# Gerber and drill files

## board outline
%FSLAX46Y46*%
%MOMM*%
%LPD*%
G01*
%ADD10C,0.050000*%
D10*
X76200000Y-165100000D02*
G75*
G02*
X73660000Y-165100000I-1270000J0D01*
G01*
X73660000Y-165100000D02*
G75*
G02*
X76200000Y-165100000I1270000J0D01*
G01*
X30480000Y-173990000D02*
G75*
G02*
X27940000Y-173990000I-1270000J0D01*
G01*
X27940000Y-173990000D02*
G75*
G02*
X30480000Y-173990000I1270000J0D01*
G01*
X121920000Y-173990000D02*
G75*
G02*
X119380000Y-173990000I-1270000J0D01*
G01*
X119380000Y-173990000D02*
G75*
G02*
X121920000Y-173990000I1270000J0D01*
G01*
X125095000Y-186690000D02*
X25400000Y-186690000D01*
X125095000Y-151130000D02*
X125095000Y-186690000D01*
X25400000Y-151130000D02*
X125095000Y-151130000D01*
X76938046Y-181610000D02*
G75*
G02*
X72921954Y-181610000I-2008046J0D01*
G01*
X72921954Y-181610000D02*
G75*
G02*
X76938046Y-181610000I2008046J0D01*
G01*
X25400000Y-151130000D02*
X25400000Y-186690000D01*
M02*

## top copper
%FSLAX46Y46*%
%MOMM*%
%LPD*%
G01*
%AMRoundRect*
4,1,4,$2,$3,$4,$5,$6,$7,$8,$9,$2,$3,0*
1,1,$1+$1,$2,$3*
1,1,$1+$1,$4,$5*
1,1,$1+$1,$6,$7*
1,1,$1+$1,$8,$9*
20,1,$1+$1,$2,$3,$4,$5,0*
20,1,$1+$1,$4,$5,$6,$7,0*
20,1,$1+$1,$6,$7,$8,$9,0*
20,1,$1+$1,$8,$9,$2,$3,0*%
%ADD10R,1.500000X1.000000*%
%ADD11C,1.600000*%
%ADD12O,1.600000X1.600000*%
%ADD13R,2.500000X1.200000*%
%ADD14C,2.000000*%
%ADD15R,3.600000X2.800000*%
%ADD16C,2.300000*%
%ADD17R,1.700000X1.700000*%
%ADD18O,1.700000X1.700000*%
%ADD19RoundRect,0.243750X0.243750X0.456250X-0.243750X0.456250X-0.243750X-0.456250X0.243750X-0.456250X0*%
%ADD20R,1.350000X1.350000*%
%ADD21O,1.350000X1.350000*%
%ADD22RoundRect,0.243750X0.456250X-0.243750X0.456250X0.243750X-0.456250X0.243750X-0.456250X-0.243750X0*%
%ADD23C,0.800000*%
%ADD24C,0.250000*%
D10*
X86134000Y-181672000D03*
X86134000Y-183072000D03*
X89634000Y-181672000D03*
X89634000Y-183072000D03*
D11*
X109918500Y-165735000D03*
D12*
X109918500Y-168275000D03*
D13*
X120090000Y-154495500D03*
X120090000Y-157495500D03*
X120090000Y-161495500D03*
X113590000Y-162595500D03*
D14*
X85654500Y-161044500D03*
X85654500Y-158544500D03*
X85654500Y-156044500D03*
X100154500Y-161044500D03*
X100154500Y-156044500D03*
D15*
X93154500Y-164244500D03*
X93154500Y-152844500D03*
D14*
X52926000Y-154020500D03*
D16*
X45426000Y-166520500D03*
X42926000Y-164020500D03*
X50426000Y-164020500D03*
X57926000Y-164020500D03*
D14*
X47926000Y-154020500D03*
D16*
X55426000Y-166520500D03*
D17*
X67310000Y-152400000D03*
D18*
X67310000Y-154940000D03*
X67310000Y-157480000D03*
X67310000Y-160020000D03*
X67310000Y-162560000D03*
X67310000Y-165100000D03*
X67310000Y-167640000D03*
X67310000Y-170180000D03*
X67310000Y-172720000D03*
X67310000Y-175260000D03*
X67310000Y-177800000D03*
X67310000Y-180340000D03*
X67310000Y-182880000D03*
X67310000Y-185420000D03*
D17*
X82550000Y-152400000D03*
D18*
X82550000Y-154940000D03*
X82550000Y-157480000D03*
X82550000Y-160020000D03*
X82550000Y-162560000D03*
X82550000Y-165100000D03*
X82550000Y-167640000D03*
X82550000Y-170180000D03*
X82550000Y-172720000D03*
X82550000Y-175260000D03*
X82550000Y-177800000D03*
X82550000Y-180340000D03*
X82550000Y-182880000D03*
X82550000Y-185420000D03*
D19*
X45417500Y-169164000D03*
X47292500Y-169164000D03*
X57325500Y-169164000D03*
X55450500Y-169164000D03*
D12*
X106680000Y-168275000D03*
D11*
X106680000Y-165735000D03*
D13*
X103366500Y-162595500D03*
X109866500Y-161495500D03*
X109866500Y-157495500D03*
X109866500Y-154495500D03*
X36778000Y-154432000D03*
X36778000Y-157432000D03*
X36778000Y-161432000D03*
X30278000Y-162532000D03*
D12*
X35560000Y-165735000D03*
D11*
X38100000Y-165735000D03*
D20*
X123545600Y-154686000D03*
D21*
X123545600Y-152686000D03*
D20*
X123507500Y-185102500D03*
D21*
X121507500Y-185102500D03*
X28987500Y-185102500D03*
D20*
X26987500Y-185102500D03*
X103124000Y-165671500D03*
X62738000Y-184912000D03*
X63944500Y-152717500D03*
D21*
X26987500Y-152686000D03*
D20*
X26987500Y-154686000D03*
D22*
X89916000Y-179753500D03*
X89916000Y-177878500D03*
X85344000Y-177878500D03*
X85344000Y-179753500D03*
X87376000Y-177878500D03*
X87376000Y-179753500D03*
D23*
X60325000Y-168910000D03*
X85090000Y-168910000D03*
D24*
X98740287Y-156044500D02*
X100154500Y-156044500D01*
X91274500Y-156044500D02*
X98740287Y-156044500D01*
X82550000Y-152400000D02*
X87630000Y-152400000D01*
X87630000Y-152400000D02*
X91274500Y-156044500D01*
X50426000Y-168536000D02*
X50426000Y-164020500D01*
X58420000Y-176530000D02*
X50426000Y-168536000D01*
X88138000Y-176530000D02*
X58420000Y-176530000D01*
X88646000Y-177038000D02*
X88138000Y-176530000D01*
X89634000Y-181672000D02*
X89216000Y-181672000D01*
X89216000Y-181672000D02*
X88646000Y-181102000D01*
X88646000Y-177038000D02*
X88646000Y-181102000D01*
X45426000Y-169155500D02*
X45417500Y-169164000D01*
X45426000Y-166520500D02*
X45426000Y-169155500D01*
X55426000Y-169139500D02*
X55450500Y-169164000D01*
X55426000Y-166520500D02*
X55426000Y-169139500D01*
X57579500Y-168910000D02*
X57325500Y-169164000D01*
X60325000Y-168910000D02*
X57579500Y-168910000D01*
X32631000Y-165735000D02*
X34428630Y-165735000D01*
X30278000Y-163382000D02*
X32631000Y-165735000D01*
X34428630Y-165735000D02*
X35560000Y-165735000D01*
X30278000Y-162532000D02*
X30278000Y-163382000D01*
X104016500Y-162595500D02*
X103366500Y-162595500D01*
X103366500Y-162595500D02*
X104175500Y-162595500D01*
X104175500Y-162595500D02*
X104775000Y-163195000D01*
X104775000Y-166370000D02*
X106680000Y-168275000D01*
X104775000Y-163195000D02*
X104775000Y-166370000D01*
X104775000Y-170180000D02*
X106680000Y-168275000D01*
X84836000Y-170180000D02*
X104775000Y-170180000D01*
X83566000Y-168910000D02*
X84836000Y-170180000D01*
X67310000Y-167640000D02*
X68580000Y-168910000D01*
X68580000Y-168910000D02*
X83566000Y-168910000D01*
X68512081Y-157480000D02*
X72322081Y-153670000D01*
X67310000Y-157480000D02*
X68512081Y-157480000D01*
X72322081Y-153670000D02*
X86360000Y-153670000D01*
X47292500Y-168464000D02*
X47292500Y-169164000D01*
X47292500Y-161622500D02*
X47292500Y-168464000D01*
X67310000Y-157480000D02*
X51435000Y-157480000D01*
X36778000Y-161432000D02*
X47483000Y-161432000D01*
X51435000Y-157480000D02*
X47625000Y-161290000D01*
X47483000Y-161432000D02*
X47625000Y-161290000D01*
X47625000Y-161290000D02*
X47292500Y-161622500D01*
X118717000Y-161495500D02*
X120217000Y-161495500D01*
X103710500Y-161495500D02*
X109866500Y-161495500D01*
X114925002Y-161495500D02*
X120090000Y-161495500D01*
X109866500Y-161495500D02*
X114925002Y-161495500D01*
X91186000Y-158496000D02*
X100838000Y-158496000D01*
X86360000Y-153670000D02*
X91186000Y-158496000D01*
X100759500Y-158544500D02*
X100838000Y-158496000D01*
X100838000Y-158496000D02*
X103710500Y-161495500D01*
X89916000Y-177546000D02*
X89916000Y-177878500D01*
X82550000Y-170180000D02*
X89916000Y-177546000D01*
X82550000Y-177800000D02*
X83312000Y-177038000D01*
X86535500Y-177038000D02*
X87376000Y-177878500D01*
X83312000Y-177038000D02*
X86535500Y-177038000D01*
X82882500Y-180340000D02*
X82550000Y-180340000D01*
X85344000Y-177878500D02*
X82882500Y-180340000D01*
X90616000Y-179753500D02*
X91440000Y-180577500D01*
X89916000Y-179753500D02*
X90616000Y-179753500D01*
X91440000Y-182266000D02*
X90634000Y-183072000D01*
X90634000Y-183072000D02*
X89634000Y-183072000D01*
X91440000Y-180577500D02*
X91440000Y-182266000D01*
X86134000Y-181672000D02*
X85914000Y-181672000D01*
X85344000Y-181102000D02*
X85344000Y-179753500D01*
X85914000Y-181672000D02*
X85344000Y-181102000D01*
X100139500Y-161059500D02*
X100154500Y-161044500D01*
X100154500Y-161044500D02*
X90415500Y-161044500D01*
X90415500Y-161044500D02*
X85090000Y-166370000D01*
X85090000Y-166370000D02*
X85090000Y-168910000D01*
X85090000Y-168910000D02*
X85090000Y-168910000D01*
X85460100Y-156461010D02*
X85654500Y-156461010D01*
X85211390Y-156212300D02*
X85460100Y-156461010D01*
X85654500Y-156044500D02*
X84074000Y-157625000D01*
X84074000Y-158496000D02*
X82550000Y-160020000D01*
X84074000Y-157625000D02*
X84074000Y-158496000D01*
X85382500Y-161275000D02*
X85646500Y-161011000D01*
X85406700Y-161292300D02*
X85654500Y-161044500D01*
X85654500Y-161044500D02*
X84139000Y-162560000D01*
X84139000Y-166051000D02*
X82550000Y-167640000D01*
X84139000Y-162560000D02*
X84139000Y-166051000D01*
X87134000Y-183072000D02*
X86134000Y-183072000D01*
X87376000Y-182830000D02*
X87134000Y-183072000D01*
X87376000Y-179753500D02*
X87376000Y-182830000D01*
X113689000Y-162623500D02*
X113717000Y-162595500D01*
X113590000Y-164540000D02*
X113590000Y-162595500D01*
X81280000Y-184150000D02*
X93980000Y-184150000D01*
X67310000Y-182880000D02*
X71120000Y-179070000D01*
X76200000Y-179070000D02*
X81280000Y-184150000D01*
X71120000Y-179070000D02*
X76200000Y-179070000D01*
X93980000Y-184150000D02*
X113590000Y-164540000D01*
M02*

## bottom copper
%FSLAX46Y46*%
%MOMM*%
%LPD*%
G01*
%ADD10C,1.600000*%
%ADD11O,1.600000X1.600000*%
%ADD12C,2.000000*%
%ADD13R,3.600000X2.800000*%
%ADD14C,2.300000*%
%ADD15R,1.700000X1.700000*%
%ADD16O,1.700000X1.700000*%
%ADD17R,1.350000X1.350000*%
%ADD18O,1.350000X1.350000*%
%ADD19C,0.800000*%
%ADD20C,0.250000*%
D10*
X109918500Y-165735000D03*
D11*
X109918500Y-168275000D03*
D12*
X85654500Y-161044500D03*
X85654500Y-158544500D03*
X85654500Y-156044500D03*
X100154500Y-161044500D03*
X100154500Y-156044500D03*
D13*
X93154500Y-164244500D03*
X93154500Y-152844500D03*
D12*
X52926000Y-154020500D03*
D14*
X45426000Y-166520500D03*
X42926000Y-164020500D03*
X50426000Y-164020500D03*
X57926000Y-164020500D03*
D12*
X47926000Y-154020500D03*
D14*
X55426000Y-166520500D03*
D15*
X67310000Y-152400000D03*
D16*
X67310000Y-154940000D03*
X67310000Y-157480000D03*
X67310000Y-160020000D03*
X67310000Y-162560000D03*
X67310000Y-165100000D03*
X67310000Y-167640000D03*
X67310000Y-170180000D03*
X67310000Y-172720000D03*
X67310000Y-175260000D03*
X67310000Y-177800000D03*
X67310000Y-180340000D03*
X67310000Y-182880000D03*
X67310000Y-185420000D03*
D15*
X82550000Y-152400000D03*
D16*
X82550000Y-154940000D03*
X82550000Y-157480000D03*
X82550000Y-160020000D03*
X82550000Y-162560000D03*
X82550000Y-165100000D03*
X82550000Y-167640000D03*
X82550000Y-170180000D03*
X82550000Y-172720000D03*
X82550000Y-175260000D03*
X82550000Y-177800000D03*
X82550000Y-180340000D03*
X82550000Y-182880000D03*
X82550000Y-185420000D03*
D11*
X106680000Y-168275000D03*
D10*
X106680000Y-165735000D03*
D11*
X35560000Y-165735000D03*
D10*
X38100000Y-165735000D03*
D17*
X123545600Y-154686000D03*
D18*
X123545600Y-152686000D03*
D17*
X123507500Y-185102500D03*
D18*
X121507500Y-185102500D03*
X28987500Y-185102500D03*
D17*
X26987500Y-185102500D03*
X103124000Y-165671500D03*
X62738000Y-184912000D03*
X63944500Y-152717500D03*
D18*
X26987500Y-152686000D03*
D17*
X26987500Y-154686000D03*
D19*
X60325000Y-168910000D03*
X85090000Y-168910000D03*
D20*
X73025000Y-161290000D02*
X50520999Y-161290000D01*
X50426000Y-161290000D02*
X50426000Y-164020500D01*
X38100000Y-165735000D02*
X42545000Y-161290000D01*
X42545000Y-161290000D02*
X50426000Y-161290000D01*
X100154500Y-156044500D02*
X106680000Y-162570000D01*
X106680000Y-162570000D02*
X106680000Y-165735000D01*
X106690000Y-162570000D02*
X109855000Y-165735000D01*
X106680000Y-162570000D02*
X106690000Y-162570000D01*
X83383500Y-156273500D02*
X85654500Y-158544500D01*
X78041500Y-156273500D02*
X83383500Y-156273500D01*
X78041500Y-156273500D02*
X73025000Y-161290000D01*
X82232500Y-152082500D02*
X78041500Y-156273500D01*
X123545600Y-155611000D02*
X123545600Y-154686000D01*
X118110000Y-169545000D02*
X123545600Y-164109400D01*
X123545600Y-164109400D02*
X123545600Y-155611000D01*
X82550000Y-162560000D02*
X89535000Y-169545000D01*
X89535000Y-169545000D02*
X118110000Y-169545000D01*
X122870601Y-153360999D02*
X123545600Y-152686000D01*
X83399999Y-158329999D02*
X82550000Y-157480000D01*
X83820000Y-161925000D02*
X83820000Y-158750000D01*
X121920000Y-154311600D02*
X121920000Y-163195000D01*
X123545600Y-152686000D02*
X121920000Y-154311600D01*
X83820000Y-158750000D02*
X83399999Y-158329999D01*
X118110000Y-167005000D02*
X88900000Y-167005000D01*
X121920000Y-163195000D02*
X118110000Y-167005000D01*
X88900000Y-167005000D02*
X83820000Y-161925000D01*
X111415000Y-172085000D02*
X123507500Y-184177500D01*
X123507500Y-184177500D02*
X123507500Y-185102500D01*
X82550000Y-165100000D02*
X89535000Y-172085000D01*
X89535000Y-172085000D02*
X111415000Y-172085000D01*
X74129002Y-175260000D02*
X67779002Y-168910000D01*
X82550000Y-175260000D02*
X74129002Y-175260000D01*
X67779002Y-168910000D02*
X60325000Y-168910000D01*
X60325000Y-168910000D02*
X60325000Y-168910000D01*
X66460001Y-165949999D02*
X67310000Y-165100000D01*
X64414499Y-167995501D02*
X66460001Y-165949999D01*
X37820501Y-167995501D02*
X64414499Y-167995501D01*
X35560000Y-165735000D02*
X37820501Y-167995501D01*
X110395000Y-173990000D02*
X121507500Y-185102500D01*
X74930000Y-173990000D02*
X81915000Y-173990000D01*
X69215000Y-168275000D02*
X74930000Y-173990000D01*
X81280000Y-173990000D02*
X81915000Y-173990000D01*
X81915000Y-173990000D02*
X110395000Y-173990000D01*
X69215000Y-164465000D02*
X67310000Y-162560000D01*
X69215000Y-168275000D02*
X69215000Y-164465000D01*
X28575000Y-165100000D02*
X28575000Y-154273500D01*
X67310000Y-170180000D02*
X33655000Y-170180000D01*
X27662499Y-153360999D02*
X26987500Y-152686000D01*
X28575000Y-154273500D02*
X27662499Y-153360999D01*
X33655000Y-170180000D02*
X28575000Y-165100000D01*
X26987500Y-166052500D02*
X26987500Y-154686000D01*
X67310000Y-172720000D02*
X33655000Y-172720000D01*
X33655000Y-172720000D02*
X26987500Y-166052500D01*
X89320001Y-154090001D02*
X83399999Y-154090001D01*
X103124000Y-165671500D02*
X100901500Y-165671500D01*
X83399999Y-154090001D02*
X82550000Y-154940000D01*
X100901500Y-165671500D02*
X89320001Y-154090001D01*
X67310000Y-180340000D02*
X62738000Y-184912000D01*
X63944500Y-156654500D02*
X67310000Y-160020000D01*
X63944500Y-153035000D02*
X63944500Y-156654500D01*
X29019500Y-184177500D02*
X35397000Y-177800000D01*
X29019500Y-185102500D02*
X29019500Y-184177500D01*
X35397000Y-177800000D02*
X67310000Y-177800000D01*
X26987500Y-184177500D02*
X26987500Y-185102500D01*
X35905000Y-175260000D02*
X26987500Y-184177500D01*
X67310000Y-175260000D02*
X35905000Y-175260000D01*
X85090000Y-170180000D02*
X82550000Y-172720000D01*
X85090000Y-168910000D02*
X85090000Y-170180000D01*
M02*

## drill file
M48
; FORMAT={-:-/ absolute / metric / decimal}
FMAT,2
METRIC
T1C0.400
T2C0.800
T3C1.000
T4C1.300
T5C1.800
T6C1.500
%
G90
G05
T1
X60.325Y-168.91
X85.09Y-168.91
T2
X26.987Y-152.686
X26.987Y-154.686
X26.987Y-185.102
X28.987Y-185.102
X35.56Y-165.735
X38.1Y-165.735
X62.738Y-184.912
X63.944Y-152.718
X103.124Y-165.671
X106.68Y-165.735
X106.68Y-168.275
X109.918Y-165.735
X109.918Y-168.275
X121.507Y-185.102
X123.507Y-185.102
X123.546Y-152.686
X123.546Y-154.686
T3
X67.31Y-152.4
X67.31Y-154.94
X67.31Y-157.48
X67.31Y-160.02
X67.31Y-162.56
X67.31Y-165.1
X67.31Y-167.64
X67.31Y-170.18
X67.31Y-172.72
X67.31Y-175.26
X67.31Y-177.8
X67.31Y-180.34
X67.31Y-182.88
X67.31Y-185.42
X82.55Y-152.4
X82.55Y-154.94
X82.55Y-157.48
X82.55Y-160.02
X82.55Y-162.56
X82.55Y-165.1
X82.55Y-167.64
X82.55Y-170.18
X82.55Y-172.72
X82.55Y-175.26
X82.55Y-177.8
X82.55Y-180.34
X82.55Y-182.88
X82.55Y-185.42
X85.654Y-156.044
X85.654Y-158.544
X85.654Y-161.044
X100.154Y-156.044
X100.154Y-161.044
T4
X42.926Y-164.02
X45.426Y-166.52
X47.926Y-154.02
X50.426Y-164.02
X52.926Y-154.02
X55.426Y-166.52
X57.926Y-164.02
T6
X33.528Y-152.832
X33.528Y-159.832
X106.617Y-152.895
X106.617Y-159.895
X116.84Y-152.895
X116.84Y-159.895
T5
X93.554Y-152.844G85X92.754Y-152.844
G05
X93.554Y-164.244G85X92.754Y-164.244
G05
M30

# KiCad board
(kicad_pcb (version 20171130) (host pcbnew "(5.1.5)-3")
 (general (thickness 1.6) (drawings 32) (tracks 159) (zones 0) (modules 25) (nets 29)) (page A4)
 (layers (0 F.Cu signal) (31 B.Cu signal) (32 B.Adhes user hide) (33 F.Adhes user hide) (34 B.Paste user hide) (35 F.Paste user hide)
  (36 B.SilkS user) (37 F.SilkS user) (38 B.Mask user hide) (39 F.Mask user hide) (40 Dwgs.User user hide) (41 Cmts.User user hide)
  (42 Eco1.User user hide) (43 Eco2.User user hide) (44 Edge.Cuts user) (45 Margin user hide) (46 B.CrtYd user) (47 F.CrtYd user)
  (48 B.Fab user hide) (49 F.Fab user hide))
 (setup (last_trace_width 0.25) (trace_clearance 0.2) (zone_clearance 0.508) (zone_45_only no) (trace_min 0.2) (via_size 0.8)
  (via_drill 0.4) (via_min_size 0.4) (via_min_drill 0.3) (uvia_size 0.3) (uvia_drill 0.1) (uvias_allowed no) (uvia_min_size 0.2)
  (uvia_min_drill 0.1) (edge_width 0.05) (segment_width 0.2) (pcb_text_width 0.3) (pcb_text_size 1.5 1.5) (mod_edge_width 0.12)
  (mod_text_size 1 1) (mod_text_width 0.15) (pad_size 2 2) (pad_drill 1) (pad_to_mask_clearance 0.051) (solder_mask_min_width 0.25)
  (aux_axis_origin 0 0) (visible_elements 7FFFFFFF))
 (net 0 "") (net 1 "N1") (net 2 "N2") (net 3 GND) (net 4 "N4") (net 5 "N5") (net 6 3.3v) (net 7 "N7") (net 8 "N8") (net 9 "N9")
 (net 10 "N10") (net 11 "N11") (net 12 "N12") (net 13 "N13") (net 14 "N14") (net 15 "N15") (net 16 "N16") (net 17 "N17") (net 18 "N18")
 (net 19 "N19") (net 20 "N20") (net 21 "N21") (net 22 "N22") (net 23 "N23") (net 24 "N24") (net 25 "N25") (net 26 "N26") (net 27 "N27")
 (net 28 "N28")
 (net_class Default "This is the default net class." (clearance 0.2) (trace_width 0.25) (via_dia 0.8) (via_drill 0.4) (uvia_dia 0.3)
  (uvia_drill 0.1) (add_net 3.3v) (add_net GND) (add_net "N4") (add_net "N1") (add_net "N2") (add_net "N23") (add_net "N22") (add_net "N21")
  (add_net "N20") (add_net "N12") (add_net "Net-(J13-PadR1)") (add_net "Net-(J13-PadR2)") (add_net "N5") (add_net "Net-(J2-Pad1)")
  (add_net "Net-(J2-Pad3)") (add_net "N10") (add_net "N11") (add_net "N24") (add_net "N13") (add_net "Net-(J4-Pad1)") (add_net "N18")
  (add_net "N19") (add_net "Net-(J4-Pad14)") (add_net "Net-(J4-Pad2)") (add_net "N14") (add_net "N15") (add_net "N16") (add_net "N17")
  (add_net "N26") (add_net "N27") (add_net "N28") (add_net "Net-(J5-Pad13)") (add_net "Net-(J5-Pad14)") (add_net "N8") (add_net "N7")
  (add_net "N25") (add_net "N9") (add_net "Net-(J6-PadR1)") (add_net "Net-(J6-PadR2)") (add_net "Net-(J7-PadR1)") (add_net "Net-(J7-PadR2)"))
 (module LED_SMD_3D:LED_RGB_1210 (layer F.Cu) (at 87.884 182.372 180)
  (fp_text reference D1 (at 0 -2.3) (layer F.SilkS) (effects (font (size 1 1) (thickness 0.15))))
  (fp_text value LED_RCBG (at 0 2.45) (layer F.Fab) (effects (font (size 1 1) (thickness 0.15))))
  (pad 3 smd rect (at 1.75 0.7) (size 1.5 1) (layers F.Cu F.Paste F.Mask) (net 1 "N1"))
  (pad 4 smd rect (at 1.75 -0.7) (size 1.5 1) (layers F.Cu F.Paste F.Mask) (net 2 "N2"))
  (pad 2 smd rect (at -1.75 0.7) (size 1.5 1) (layers F.Cu F.Paste F.Mask) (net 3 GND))
  (pad 1 smd rect (at -1.75 -0.7) (size 1.5 1) (layers F.Cu F.Paste F.Mask) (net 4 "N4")))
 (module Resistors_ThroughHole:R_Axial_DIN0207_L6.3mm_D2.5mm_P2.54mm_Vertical (layer F.Cu) (at 109.9185 165.735 270)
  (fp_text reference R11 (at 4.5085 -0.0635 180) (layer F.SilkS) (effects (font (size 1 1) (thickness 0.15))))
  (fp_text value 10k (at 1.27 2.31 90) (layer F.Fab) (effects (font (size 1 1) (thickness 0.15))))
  (pad 1 thru_hole circle (at 0 0 270) (size 1.6 1.6) (drill 0.8) (layers *.Cu *.Mask) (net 3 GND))
  (pad 2 thru_hole oval (at 2.54 0 270) (size 1.6 1.6) (drill 0.8) (layers *.Cu *.Mask) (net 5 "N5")))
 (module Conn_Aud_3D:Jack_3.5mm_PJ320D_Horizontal (layer F.Cu) (at 116.84 157.6705 270)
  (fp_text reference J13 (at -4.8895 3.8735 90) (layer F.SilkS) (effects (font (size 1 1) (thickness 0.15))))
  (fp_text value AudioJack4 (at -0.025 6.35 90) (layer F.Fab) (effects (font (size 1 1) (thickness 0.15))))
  (pad "" np_thru_hole circle (at 2.225 0 270) (size 1.5 1.5) (drill 1.5) (layers *.Cu *.Mask))
  (pad "" np_thru_hole circle (at -4.775 0 270) (size 1.5 1.5) (drill 1.5) (layers *.Cu *.Mask))
  (pad R2 smd rect (at -3.175 -3.25 270) (size 1.2 2.5) (layers F.Cu F.Paste F.Mask))
  (pad R1 smd rect (at -0.175 -3.25 270) (size 1.2 2.5) (layers F.Cu F.Paste F.Mask))
  (pad T smd rect (at 3.825 -3.25 270) (size 1.2 2.5) (layers F.Cu F.Paste F.Mask) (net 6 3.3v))
  (pad S smd rect (at 4.925 3.25 270) (size 1.2 2.5) (layers F.Cu F.Paste F.Mask) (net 5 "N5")))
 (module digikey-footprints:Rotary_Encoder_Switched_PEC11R (layer F.Cu) (at 93.1545 152.8445 270)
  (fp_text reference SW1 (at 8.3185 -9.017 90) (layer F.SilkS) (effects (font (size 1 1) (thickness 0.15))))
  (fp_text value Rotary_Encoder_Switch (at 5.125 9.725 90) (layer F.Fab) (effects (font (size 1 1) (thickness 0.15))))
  (pad B thru_hole circle (at 8.2 7.5 270) (size 2 2) (drill 1) (layers *.Cu *.Mask) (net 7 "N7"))
  (pad C thru_hole circle (at 5.7 7.5 270) (size 2 2) (drill 1) (layers *.Cu *.Mask) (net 3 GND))
  (pad A thru_hole circle (at 3.2 7.5 270) (size 2 2) (drill 1) (layers *.Cu *.Mask) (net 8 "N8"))
  (pad S2 thru_hole circle (at 8.2 -7 270) (size 2 2) (drill 1) (layers *.Cu *.Mask) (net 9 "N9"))
  (pad S1 thru_hole circle (at 3.2 -7 270) (size 2 2) (drill 1) (layers *.Cu *.Mask) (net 3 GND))
  (pad 3 thru_hole rect (at 11.4 0 270) (size 2.8 3.6) (drill oval 1.8 2.6) (layers *.Cu *.Mask))
  (pad 3 thru_hole rect (at 0 0 270) (size 2.8 3.6) (drill oval 1.8 2.6) (layers *.Cu *.Mask)))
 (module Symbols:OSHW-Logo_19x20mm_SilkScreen (layer F.Cu) (at 110.49 175.895)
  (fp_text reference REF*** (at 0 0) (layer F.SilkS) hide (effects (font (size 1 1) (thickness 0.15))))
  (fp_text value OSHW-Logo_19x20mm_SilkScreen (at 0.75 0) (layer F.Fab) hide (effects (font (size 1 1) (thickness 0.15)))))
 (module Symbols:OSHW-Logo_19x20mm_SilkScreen (layer B.Cu) (at 110.49 175.895 180)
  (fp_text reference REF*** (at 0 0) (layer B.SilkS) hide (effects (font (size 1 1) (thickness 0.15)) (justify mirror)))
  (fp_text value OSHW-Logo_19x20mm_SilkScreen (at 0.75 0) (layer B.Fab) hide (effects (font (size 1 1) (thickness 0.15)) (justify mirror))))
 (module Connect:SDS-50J (layer F.Cu) (at 42.926 164.0205)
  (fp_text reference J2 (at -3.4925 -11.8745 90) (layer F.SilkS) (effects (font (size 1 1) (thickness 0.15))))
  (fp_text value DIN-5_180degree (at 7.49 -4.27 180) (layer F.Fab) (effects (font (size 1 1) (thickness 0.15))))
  (pad "" thru_hole circle (at 10 -10) (size 2 2) (drill 1.3) (layers *.Cu *.Mask))
  (pad 4 thru_hole circle (at 2.5 2.5) (size 2.3 2.3) (drill 1.3) (layers *.Cu *.Mask) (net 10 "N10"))
  (pad 1 thru_hole circle (at 0 0) (size 2.3 2.3) (drill 1.3) (layers *.Cu *.Mask))
  (pad 2 thru_hole circle (at 7.5 0) (size 2.3 2.3) (drill 1.3) (layers *.Cu *.Mask) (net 3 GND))
  (pad 3 thru_hole circle (at 15 0) (size 2.3 2.3) (drill 1.3) (layers *.Cu *.Mask))
  (pad "" thru_hole circle (at 5 -10) (size 2 2) (drill 1.3) (layers *.Cu *.Mask))
  (pad 5 thru_hole circle (at 12.5 2.5) (size 2.3 2.3) (drill 1.3) (layers *.Cu *.Mask) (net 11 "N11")))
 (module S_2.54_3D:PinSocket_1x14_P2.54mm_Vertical (layer F.Cu) (at 67.31 152.4)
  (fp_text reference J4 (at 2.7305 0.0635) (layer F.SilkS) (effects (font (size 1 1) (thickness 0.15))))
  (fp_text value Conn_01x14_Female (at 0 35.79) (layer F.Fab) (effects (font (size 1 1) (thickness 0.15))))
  (pad 1 thru_hole rect (at 0 0) (size 1.7 1.7) (drill 1) (layers *.Cu *.Mask))
  (pad 2 thru_hole oval (at 0 2.54) (size 1.7 1.7) (drill 1) (layers *.Cu *.Mask))
  (pad 3 thru_hole oval (at 0 5.08) (size 1.7 1.7) (drill 1) (layers *.Cu *.Mask) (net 6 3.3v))
  (pad 4 thru_hole oval (at 0 7.62) (size 1.7 1.7) (drill 1) (layers *.Cu *.Mask) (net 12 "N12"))
  (pad 5 thru_hole oval (at 0 10.16) (size 1.7 1.7) (drill 1) (layers *.Cu *.Mask) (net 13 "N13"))
  (pad 6 thru_hole oval (at 0 12.7) (size 1.7 1.7) (drill 1) (layers *.Cu *.Mask) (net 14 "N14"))
  (pad 7 thru_hole oval (at 0 15.24) (size 1.7 1.7) (drill 1) (layers *.Cu *.Mask) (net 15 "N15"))
  (pad 8 thru_hole oval (at 0 17.78) (size 1.7 1.7) (drill 1) (layers *.Cu *.Mask) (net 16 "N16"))
  (pad 9 thru_hole oval (at 0 20.32) (size 1.7 1.7) (drill 1) (layers *.Cu *.Mask) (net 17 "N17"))
  (pad 10 thru_hole oval (at 0 22.86) (size 1.7 1.7) (drill 1) (layers *.Cu *.Mask) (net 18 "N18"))
  (pad 11 thru_hole oval (at 0 25.4) (size 1.7 1.7) (drill 1) (layers *.Cu *.Mask) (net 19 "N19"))
  (pad 12 thru_hole oval (at 0 27.94) (size 1.7 1.7) (drill 1) (layers *.Cu *.Mask) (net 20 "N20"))
  (pad 13 thru_hole oval (at 0 30.48) (size 1.7 1.7) (drill 1) (layers *.Cu *.Mask) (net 5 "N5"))
  (pad 14 thru_hole oval (at 0 33.02) (size 1.7 1.7) (drill 1) (layers *.Cu *.Mask)))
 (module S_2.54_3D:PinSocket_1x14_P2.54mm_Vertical (layer F.Cu) (at 82.55 152.4)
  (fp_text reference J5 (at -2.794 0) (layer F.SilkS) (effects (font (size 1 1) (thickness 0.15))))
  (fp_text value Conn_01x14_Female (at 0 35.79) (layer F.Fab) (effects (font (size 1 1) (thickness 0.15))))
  (pad 1 thru_hole rect (at 0 0) (size 1.7 1.7) (drill 1) (layers *.Cu *.Mask) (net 3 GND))
  (pad 2 thru_hole oval (at 0 2.54) (size 1.7 1.7) (drill 1) (layers *.Cu *.Mask) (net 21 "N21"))
  (pad 3 thru_hole oval (at 0 5.08) (size 1.7 1.7) (drill 1) (layers *.Cu *.Mask) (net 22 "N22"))
  (pad 4 thru_hole oval (at 0 7.62) (size 1.7 1.7) (drill 1) (layers *.Cu *.Mask) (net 8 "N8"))
  (pad 5 thru_hole oval (at 0 10.16) (size 1.7 1.7) (drill 1) (layers *.Cu *.Mask) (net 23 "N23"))
  (pad 6 thru_hole oval (at 0 12.7) (size 1.7 1.7) (drill 1) (layers *.Cu *.Mask) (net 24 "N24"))
  (pad 7 thru_hole oval (at 0 15.24) (size 1.7 1.7) (drill 1) (layers *.Cu *.Mask) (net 7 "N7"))
  (pad 8 thru_hole oval (at 0 17.78) (size 1.7 1.7) (drill 1) (layers *.Cu *.Mask) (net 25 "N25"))
  (pad 9 thru_hole oval (at 0 20.32) (size 1.7 1.7) (drill 1) (layers *.Cu *.Mask) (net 9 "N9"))
  (pad 10 thru_hole oval (at 0 22.86) (size 1.7 1.7) (drill 1) (layers *.Cu *.Mask) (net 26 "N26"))
  (pad 11 thru_hole oval (at 0 25.4) (size 1.7 1.7) (drill 1) (layers *.Cu *.Mask) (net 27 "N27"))
  (pad 12 thru_hole oval (at 0 27.94) (size 1.7 1.7) (drill 1) (layers *.Cu *.Mask) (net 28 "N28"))
  (pad 13 thru_hole oval (at 0 30.48) (size 1.7 1.7) (drill 1) (layers *.Cu *.Mask))
  (pad 14 thru_hole oval (at 0 33.02) (size 1.7 1.7) (drill 1) (layers *.Cu *.Mask)))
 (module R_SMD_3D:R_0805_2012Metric (layer F.Cu) (at 46.355 169.164 180)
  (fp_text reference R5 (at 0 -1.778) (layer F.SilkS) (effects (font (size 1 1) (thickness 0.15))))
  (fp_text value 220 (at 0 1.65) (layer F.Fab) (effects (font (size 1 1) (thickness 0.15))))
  (pad 2 smd roundrect (at 0.9375 0 180) (size 0.975 1.4) (layers F.Cu F.Paste F.Mask) (roundrect_rratio 0.25) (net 10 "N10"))
  (pad 1 smd roundrect (at -0.9375 0 180) (size 0.975 1.4) (layers F.Cu F.Paste F.Mask) (roundrect_rratio 0.25) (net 6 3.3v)))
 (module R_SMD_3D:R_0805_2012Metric (layer F.Cu) (at 56.388 169.164 180)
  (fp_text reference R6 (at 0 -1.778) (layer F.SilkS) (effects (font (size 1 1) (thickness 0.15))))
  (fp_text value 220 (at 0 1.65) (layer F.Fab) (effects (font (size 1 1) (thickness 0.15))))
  (pad 1 smd roundrect (at -0.9375 0 180) (size 0.975 1.4) (layers F.Cu F.Paste F.Mask) (roundrect_rratio 0.25) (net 26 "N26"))
  (pad 2 smd roundrect (at 0.9375 0 180) (size 0.975 1.4) (layers F.Cu F.Paste F.Mask) (roundrect_rratio 0.25) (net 11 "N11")))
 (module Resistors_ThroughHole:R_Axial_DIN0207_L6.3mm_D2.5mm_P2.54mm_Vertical (layer F.Cu) (at 106.68 165.735 270)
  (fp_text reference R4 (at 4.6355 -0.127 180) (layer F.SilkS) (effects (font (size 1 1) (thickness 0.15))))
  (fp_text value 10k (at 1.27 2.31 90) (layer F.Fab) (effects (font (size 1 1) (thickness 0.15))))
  (pad 2 thru_hole oval (at 2.54 0 270) (size 1.6 1.6) (drill 0.8) (layers *.Cu *.Mask) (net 15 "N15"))
  (pad 1 thru_hole circle (at 0 0 270) (size 1.6 1.6) (drill 0.8) (layers *.Cu *.Mask) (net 3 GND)))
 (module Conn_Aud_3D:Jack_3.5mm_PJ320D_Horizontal (layer F.Cu) (at 106.6165 157.6705 270)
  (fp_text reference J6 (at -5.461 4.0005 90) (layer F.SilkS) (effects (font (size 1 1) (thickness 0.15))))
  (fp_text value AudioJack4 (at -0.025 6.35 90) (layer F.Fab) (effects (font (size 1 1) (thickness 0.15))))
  (pad S smd rect (at 4.925 3.25 270) (size 1.2 2.5) (layers F.Cu F.Paste F.Mask) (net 15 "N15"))
  (pad T smd rect (at 3.825 -3.25 270) (size 1.2 2.5) (layers F.Cu F.Paste F.Mask) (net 6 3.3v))
  (pad R1 smd rect (at -0.175 -3.25 270) (size 1.2 2.5) (layers F.Cu F.Paste F.Mask))
  (pad R2 smd rect (at -3.175 -3.25 270) (size 1.2 2.5) (layers F.Cu F.Paste F.Mask))
  (pad "" np_thru_hole circle (at -4.775 0 270) (size 1.5 1.5) (drill 1.5) (layers *.Cu *.Mask))
  (pad "" np_thru_hole circle (at 2.225 0 270) (size 1.5 1.5) (drill 1.5) (layers *.Cu *.Mask)))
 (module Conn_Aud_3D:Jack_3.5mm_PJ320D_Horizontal (layer F.Cu) (at 33.528 157.607 270)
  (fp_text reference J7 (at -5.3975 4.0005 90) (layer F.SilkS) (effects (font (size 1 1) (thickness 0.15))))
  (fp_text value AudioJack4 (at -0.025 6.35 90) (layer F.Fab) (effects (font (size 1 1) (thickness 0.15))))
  (pad "" np_thru_hole circle (at 2.225 0 270) (size 1.5 1.5) (drill 1.5) (layers *.Cu *.Mask))
  (pad "" np_thru_hole circle (at -4.775 0 270) (size 1.5 1.5) (drill 1.5) (layers *.Cu *.Mask))
  (pad R2 smd rect (at -3.175 -3.25 270) (size 1.2 2.5) (layers F.Cu F.Paste F.Mask))
  (pad R1 smd rect (at -0.175 -3.25 270) (size 1.2 2.5) (layers F.Cu F.Paste F.Mask))
  (pad T smd rect (at 3.825 -3.25 270) (size 1.2 2.5) (layers F.Cu F.Paste F.Mask) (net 6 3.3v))
  (pad S smd rect (at 4.925 3.25 270) (size 1.2 2.5) (layers F.Cu F.Paste F.Mask) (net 14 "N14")))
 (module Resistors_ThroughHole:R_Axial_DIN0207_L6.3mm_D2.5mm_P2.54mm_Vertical (layer F.Cu) (at 38.1 165.735 180)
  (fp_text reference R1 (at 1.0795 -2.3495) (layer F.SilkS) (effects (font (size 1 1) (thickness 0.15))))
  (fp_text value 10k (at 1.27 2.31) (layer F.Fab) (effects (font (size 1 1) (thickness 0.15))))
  (pad 2 thru_hole oval (at 2.54 0 180) (size 1.6 1.6) (drill 0.8) (layers *.Cu *.Mask) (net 14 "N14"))
  (pad 1 thru_hole circle (at 0 0 180) (size 1.6 1.6) (drill 0.8) (layers *.Cu *.Mask) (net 3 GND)))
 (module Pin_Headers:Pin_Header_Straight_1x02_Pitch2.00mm (layer F.Cu) (at 123.5456 154.686 180)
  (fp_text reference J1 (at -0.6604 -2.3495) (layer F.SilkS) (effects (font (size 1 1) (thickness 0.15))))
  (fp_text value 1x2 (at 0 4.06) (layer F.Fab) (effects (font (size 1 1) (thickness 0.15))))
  (pad 1 thru_hole rect (at 0 0 180) (size 1.35 1.35) (drill 0.8) (layers *.Cu *.Mask) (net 23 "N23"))
  (pad 2 thru_hole oval (at 0 2 180) (size 1.35 1.35) (drill 0.8) (layers *.Cu *.Mask) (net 22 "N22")))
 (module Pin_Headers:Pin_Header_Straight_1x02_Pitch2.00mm (layer F.Cu) (at 123.5075 185.1025 270)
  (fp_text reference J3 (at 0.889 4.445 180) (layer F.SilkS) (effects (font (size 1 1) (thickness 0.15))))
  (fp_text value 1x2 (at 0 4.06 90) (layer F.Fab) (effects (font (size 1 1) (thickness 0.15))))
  (pad 1 thru_hole rect (at 0 0 270) (size 1.35 1.35) (drill 0.8) (layers *.Cu *.Mask) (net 24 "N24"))
  (pad 2 thru_hole oval (at 0 2 270) (size 1.35 1.35) (drill 0.8) (layers *.Cu *.Mask) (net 13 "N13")))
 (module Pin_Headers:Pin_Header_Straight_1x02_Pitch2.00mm (layer F.Cu) (at 26.9875 185.1025 90)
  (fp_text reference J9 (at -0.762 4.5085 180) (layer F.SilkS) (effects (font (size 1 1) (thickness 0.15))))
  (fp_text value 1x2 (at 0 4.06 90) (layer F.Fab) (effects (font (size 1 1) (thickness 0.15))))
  (pad 2 thru_hole oval (at 0 2 90) (size 1.35 1.35) (drill 0.8) (layers *.Cu *.Mask) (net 19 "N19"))
  (pad 1 thru_hole rect (at 0 0 90) (size 1.35 1.35) (drill 0.8) (layers *.Cu *.Mask) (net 18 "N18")))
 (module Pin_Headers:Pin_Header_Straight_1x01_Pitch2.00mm (layer F.Cu) (at 103.124 165.6715)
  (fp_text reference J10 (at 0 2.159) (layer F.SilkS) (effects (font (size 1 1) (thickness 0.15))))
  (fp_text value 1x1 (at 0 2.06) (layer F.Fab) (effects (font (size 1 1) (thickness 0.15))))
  (pad 1 thru_hole rect (at 0 0) (size 1.35 1.35) (drill 0.8) (layers *.Cu *.Mask) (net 21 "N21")))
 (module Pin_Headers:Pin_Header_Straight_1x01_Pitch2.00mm (layer F.Cu) (at 62.738 184.912)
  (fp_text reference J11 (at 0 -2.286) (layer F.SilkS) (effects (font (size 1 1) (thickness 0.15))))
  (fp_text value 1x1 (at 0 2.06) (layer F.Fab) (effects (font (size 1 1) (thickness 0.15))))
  (pad 1 thru_hole rect (at 0 0) (size 1.35 1.35) (drill 0.8) (layers *.Cu *.Mask) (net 20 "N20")))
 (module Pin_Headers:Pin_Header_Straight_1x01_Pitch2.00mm (layer F.Cu) (at 63.9445 152.7175)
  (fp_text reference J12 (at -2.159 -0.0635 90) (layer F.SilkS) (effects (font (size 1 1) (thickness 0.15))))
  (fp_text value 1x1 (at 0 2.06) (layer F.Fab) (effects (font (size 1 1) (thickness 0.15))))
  (pad 1 thru_hole rect (at 0 0) (size 1.35 1.35) (drill 0.8) (layers *.Cu *.Mask) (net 12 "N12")))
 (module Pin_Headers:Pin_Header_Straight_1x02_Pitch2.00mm (layer F.Cu) (at 26.9875 154.686 180)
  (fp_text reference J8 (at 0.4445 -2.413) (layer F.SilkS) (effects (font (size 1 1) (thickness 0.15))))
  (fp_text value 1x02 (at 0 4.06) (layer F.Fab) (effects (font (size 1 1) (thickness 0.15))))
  (pad 2 thru_hole oval (at 0 2 180) (size 1.35 1.35) (drill 0.8) (layers *.Cu *.Mask) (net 16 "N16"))
  (pad 1 thru_hole rect (at 0 0 180) (size 1.35 1.35) (drill 0.8) (layers *.Cu *.Mask) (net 17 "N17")))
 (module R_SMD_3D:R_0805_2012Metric (layer F.Cu) (at 89.916 178.816 90)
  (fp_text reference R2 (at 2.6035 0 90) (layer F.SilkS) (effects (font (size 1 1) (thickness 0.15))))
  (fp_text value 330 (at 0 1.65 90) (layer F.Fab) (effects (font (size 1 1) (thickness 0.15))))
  (pad 1 smd roundrect (at -0.9375 0 90) (size 0.975 1.4) (layers F.Cu F.Paste F.Mask) (roundrect_rratio 0.25) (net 4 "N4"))
  (pad 2 smd roundrect (at 0.9375 0 90) (size 0.975 1.4) (layers F.Cu F.Paste F.Mask) (roundrect_rratio 0.25) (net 25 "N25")))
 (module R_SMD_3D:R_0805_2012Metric (layer F.Cu) (at 85.344 178.816 90)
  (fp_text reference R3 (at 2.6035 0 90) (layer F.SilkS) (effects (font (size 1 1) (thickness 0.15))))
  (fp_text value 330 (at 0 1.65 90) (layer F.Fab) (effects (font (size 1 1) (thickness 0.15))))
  (pad 2 smd roundrect (at 0.9375 0 90) (size 0.975 1.4) (layers F.Cu F.Paste F.Mask) (roundrect_rratio 0.25) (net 28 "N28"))
  (pad 1 smd roundrect (at -0.9375 0 90) (size 0.975 1.4) (layers F.Cu F.Paste F.Mask) (roundrect_rratio 0.25) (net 1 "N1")))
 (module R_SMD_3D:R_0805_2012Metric (layer F.Cu) (at 87.376 178.816 90)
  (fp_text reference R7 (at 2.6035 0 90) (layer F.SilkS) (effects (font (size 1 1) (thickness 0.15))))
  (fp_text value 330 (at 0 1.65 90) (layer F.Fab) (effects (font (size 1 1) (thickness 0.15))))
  (pad 2 smd roundrect (at 0.9375 0 90) (size 0.975 1.4) (layers F.Cu F.Paste F.Mask) (roundrect_rratio 0.25) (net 27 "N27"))
  (pad 1 smd roundrect (at -0.9375 0 90) (size 0.975 1.4) (layers F.Cu F.Paste F.Mask) (roundrect_rratio 0.25) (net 2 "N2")))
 (gr_circle (center 74.93 165.1) (end 76.2 165.1) (layer Edge.Cuts) (width 0.05))
 (gr_circle (center 29.21 173.99) (end 27.94 173.99) (layer Edge.Cuts) (width 0.05))
 (gr_circle (center 120.65 173.99) (end 121.92 173.99) (layer Edge.Cuts) (width 0.05))
 (gr_line (start 125.095 186.69) (end 25.4 186.69) (layer Edge.Cuts) (width 0.05))
 (gr_line (start 125.095 151.13) (end 125.095 186.69) (layer Edge.Cuts) (width 0.05))
 (gr_line (start 25.4 151.13) (end 125.095 151.13) (layer Edge.Cuts) (width 0.05))
 (gr_circle (center 74.93 181.61) (end 76.835 180.975) (layer Edge.Cuts) (width 0.05))
 (gr_line (start 25.4 151.13) (end 25.4 186.69) (layer Edge.Cuts) (width 0.05))
 (segment (start 98.740287 156.0445) (end 100.1545 156.0445) (width 0.25) (layer F.Cu) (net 3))
 (segment (start 91.2745 156.0445) (end 98.740287 156.0445) (width 0.25) (layer F.Cu) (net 3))
 (segment (start 82.55 152.4) (end 87.63 152.4) (width 0.25) (layer F.Cu) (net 3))
 (segment (start 87.63 152.4) (end 91.2745 156.0445) (width 0.25) (layer F.Cu) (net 3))
 (segment (start 73.025 161.29) (end 50.520999 161.29) (width 0.25) (layer B.Cu) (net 3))
 (segment (start 50.426 161.29) (end 50.426 164.0205) (width 0.25) (layer B.Cu) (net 3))
 (segment (start 38.1 165.735) (end 42.545 161.29) (width 0.25) (layer B.Cu) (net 3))
 (segment (start 42.545 161.29) (end 50.426 161.29) (width 0.25) (layer B.Cu) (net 3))
 (segment (start 100.1545 156.0445) (end 106.68 162.57) (width 0.25) (layer B.Cu) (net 3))
 (segment (start 106.68 162.57) (end 106.68 165.735) (width 0.25) (layer B.Cu) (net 3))
 (segment (start 106.69 162.57) (end 109.855 165.735) (width 0.25) (layer B.Cu) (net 3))
 (segment (start 106.68 162.57) (end 106.69 162.57) (width 0.25) (layer B.Cu) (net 3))
 (segment (start 83.3835 156.2735) (end 85.6545 158.5445) (width 0.25) (layer B.Cu) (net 3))
 (segment (start 78.0415 156.2735) (end 83.3835 156.2735) (width 0.25) (layer B.Cu) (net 3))
 (segment (start 78.0415 156.2735) (end 73.025 161.29) (width 0.25) (layer B.Cu) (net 3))
 (segment (start 82.2325 152.0825) (end 78.0415 156.2735) (width 0.25) (layer B.Cu) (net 3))
 (segment (start 50.426 168.536) (end 50.426 164.0205) (width 0.25) (layer F.Cu) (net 3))
 (segment (start 58.42 176.53) (end 50.426 168.536) (width 0.25) (layer F.Cu) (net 3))
 (segment (start 88.138 176.53) (end 58.42 176.53) (width 0.25) (layer F.Cu) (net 3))
 (segment (start 88.646 177.038) (end 88.138 176.53) (width 0.25) (layer F.Cu) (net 3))
 (segment (start 89.634 181.672) (end 89.216 181.672) (width 0.25) (layer F.Cu) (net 3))
 (segment (start 89.216 181.672) (end 88.646 181.102) (width 0.25) (layer F.Cu) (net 3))
 (segment (start 88.646 177.038) (end 88.646 181.102) (width 0.25) (layer F.Cu) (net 3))
 (segment (start 123.5456 155.611) (end 123.5456 154.686) (width 0.25) (layer B.Cu) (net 23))
 (segment (start 118.11 169.545) (end 123.5456 164.1094) (width 0.25) (layer B.Cu) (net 23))
 (segment (start 123.5456 164.1094) (end 123.5456 155.611) (width 0.25) (layer B.Cu) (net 23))
 (segment (start 82.55 162.56) (end 89.535 169.545) (width 0.25) (layer B.Cu) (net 23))
 (segment (start 89.535 169.545) (end 118.11 169.545) (width 0.25) (layer B.Cu) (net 23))
 (segment (start 122.870601 153.360999) (end 123.5456 152.686) (width 0.25) (layer B.Cu) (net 22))
 (segment (start 83.399999 158.329999) (end 82.55 157.48) (width 0.25) (layer B.Cu) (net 22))
 (segment (start 83.82 161.925) (end 83.82 158.75) (width 0.25) (layer B.Cu) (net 22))
 (segment (start 121.92 154.3116) (end 121.92 163.195) (width 0.25) (layer B.Cu) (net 22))
 (segment (start 123.5456 152.686) (end 121.92 154.3116) (width 0.25) (layer B.Cu) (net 22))
 (segment (start 83.82 158.75) (end 83.399999 158.329999) (width 0.25) (layer B.Cu) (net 22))
 (segment (start 118.11 167.005) (end 88.9 167.005) (width 0.25) (layer B.Cu) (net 22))
 (segment (start 121.92 163.195) (end 118.11 167.005) (width 0.25) (layer B.Cu) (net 22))
 (segment (start 88.9 167.005) (end 83.82 161.925) (width 0.25) (layer B.Cu) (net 22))
 (segment (start 45.426 169.1555) (end 45.4175 169.164) (width 0.25) (layer F.Cu) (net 10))
 (segment (start 45.426 166.5205) (end 45.426 169.1555) (width 0.25) (layer F.Cu) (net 10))
 (segment (start 55.426 169.1395) (end 55.4505 169.164) (width 0.25) (layer F.Cu) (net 11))
 (segment (start 55.426 166.5205) (end 55.426 169.1395) (width 0.25) (layer F.Cu) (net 11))
 (segment (start 111.415 172.085) (end 123.5075 184.1775) (width 0.25) (layer B.Cu) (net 24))
 (segment (start 123.5075 184.1775) (end 123.5075 185.1025) (width 0.25) (layer B.Cu) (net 24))
 (segment (start 82.55 165.1) (end 89.535 172.085) (width 0.25) (layer B.Cu) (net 24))
 (segment (start 89.535 172.085) (end 111.415 172.085) (width 0.25) (layer B.Cu) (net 24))
 (segment (start 74.129002 175.26) (end 67.779002 168.91) (width 0.25) (layer B.Cu) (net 26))
 (segment (start 82.55 175.26) (end 74.129002 175.26) (width 0.25) (layer B.Cu) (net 26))
 (segment (start 67.779002 168.91) (end 60.325 168.91) (width 0.25) (layer B.Cu) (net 26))
 (segment (start 60.325 168.91) (end 60.325 168.91) (width 0.25) (layer B.Cu) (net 26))
 (via (at 60.325 168.91) (size 0.8) (drill 0.4) (layers F.Cu B.Cu) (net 26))
 (segment (start 57.5795 168.91) (end 57.3255 169.164) (width 0.25) (layer F.Cu) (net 26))
 (segment (start 60.325 168.91) (end 57.5795 168.91) (width 0.25) (layer F.Cu) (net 26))
 (segment (start 32.631 165.735) (end 34.42863 165.735) (width 0.25) (layer F.Cu) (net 14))
 (segment (start 30.278 163.382) (end 32.631 165.735) (width 0.25) (layer F.Cu) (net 14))
 (segment (start 34.42863 165.735) (end 35.56 165.735) (width 0.25) (layer F.Cu) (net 14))
 (segment (start 30.278 162.532) (end 30.278 163.382) (width 0.25) (layer F.Cu) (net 14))
 (segment (start 66.460001 165.949999) (end 67.31 165.1) (width 0.25) (layer B.Cu) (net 14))
 (segment (start 64.414499 167.995501) (end 66.460001 165.949999) (width 0.25) (layer B.Cu) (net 14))
 (segment (start 37.820501 167.995501) (end 64.414499 167.995501) (width 0.25) (layer B.Cu) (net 14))
 (segment (start 35.56 165.735) (end 37.820501 167.995501) (width 0.25) (layer B.Cu) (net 14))
 (segment (start 104.0165 162.5955) (end 103.3665 162.5955) (width 0.25) (layer F.Cu) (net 15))
 (segment (start 103.3665 162.5955) (end 104.1755 162.5955) (width 0.25) (layer F.Cu) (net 15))
 (segment (start 104.1755 162.5955) (end 104.775 163.195) (width 0.25) (layer F.Cu) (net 15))
 (segment (start 104.775 166.37) (end 106.68 168.275) (width 0.25) (layer F.Cu) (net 15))
 (segment (start 104.775 163.195) (end 104.775 166.37) (width 0.25) (layer F.Cu) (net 15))
 (segment (start 104.775 170.18) (end 106.68 168.275) (width 0.25) (layer F.Cu) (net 15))
 (segment (start 84.836 170.18) (end 104.775 170.18) (width 0.25) (layer F.Cu) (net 15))
 (segment (start 83.566 168.91) (end 84.836 170.18) (width 0.25) (layer F.Cu) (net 15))
 (segment (start 67.31 167.64) (end 68.58 168.91) (width 0.25) (layer F.Cu) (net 15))
 (segment (start 68.58 168.91) (end 83.566 168.91) (width 0.25) (layer F.Cu) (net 15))
 (segment (start 110.395 173.99) (end 121.5075 185.1025) (width 0.25) (layer B.Cu) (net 13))
 (segment (start 74.93 173.99) (end 81.915 173.99) (width 0.25) (layer B.Cu) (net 13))
 (segment (start 69.215 168.275) (end 74.93 173.99) (width 0.25) (layer B.Cu) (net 13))
 (segment (start 81.28 173.99) (end 81.915 173.99) (width 0.25) (layer B.Cu) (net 13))
 (segment (start 81.915 173.99) (end 110.395 173.99) (width 0.25) (layer B.Cu) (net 13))
 (segment (start 69.215 164.465) (end 67.31 162.56) (width 0.25) (layer B.Cu) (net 13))
 (segment (start 69.215 168.275) (end 69.215 164.465) (width 0.25) (layer B.Cu) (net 13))
 (segment (start 68.512081 157.48) (end 72.322081 153.67) (width 0.25) (layer F.Cu) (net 6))
 (segment (start 67.31 157.48) (end 68.512081 157.48) (width 0.25) (layer F.Cu) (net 6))
 (segment (start 72.322081 153.67) (end 86.36 153.67) (width 0.25) (layer F.Cu) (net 6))
 (segment (start 47.2925 168.464) (end 47.2925 169.164) (width 0.25) (layer F.Cu) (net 6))
 (segment (start 47.2925 161.6225) (end 47.2925 168.464) (width 0.25) (layer F.Cu) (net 6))
 (segment (start 67.31 157.48) (end 51.435 157.48) (width 0.25) (layer F.Cu) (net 6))
 (segment (start 36.778 161.432) (end 47.483 161.432) (width 0.25) (layer F.Cu) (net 6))
 (segment (start 51.435 157.48) (end 47.625 161.29) (width 0.25) (layer F.Cu) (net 6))
 (segment (start 47.483 161.432) (end 47.625 161.29) (width 0.25) (layer F.Cu) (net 6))
 (segment (start 47.625 161.29) (end 47.2925 161.6225) (width 0.25) (layer F.Cu) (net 6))
 (segment (start 118.717 161.4955) (end 120.217 161.4955) (width 0.25) (layer F.Cu) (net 6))
 (segment (start 103.7105 161.4955) (end 109.8665 161.4955) (width 0.25) (layer F.Cu) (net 6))
 (segment (start 114.925002 161.4955) (end 120.09 161.4955) (width 0.25) (layer F.Cu) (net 6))
 (segment (start 109.8665 161.4955) (end 114.925002 161.4955) (width 0.25) (layer F.Cu) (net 6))
 (segment (start 91.186 158.496) (end 100.838 158.496) (width 0.25) (layer F.Cu) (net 6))
 (segment (start 86.36 153.67) (end 91.186 158.496) (width 0.25) (layer F.Cu) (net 6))
 (segment (start 100.7595 158.5445) (end 100.838 158.496) (width 0.25) (layer F.Cu) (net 6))
 (segment (start 100.838 158.496) (end 103.7105 161.4955) (width 0.25) (layer F.Cu) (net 6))
 (segment (start 28.575 165.1) (end 28.575 154.2735) (width 0.25) (layer B.Cu) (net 16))
 (segment (start 67.31 170.18) (end 33.655 170.18) (width 0.25) (layer B.Cu) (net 16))
 (segment (start 27.662499 153.360999) (end 26.9875 152.686) (width 0.25) (layer B.Cu) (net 16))
 (segment (start 28.575 154.2735) (end 27.662499 153.360999) (width 0.25) (layer B.Cu) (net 16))
 (segment (start 33.655 170.18) (end 28.575 165.1) (width 0.25) (layer B.Cu) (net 16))
 (segment (start 26.9875 166.0525) (end 26.9875 154.686) (width 0.25) (layer B.Cu) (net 17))
 (segment (start 67.31 172.72) (end 33.655 172.72) (width 0.25) (layer B.Cu) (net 17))
 (segment (start 33.655 172.72) (end 26.9875 166.0525) (width 0.25) (layer B.Cu) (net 17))
 (segment (start 89.320001 154.090001) (end 83.399999 154.090001) (width 0.25) (layer B.Cu) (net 21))
 (segment (start 103.124 165.6715) (end 100.9015 165.6715) (width 0.25) (layer B.Cu) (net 21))
 (segment (start 83.399999 154.090001) (end 82.55 154.94) (width 0.25) (layer B.Cu) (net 21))
 (segment (start 100.9015 165.6715) (end 89.320001 154.090001) (width 0.25) (layer B.Cu) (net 21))
 (segment (start 67.31 180.34) (end 62.738 184.912) (width 0.25) (layer B.Cu) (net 20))
 (segment (start 63.9445 156.6545) (end 67.31 160.02) (width 0.25) (layer B.Cu) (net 12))
 (segment (start 63.9445 153.035) (end 63.9445 156.6545) (width 0.25) (layer B.Cu) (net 12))
 (segment (start 89.916 177.546) (end 89.916 177.8785) (width 0.25) (layer F.Cu) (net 25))
 (segment (start 82.55 170.18) (end 89.916 177.546) (width 0.25) (layer F.Cu) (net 25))
 (segment (start 82.55 177.8) (end 83.312 177.038) (width 0.25) (layer F.Cu) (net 27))
 (segment (start 86.5355 177.038) (end 87.376 177.8785) (width 0.25) (layer F.Cu) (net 27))
 (segment (start 83.312 177.038) (end 86.5355 177.038) (width 0.25) (layer F.Cu) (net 27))
 (segment (start 82.8825 180.34) (end 82.55 180.34) (width 0.25) (layer F.Cu) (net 28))
 (segment (start 85.344 177.8785) (end 82.8825 180.34) (width 0.25) (layer F.Cu) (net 28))
 (segment (start 29.0195 184.1775) (end 35.397 177.8) (width 0.25) (layer B.Cu) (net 19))
 (segment (start 29.0195 185.1025) (end 29.0195 184.1775) (width 0.25) (layer B.Cu) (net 19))
 (segment (start 35.397 177.8) (end 67.31 177.8) (width 0.25) (layer B.Cu) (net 19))
 (segment (start 26.9875 184.1775) (end 26.9875 185.1025) (width 0.25) (layer B.Cu) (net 18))
 (segment (start 35.905 175.26) (end 26.9875 184.1775) (width 0.25) (layer B.Cu) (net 18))
 (segment (start 67.31 175.26) (end 35.905 175.26) (width 0.25) (layer B.Cu) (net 18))
 (segment (start 90.616 179.7535) (end 91.44 180.5775) (width 0.25) (layer F.Cu) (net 4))
 (segment (start 89.916 179.7535) (end 90.616 179.7535) (width 0.25) (layer F.Cu) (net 4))
 (segment (start 91.44 182.266) (end 90.634 183.072) (width 0.25) (layer F.Cu) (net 4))
 (segment (start 90.634 183.072) (end 89.634 183.072) (width 0.25) (layer F.Cu) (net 4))
 (segment (start 91.44 180.5775) (end 91.44 182.266) (width 0.25) (layer F.Cu) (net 4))
 (segment (start 86.134 181.672) (end 85.914 181.672) (width 0.25) (layer F.Cu) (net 1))
 (segment (start 85.344 181.102) (end 85.344 179.7535) (width 0.25) (layer F.Cu) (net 1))
 (segment (start 85.914 181.672) (end 85.344 181.102) (width 0.25) (layer F.Cu) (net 1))
 (segment (start 100.1395 161.0595) (end 100.1545 161.0445) (width 0.25) (layer F.Cu) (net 9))
 (segment (start 100.1545 161.0445) (end 90.4155 161.0445) (width 0.25) (layer F.Cu) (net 9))
 (segment (start 90.4155 161.0445) (end 85.09 166.37) (width 0.25) (layer F.Cu) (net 9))
 (segment (start 85.09 166.37) (end 85.09 168.91) (width 0.25) (layer F.Cu) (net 9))
 (segment (start 85.09 168.91) (end 85.09 168.91) (width 0.25) (layer F.Cu) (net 9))
 (via (at 85.09 168.91) (size 0.8) (drill 0.4) (layers F.Cu B.Cu) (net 9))
 (segment (start 85.09 170.18) (end 82.55 172.72) (width 0.25) (layer B.Cu) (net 9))
 (segment (start 85.09 168.91) (end 85.09 170.18) (width 0.25) (layer B.Cu) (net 9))
 (segment (start 85.4601 156.46101) (end 85.6545 156.46101) (width 0.25) (layer F.Cu) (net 8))
 (segment (start 85.21139 156.2123) (end 85.4601 156.46101) (width 0.25) (layer F.Cu) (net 8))
 (segment (start 85.6545 156.0445) (end 84.074 157.625) (width 0.25) (layer F.Cu) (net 8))
 (segment (start 84.074 158.496) (end 82.55 160.02) (width 0.25) (layer F.Cu) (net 8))
 (segment (start 84.074 157.625) (end 84.074 158.496) (width 0.25) (layer F.Cu) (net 8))
 (segment (start 85.3825 161.275) (end 85.6465 161.011) (width 0.25) (layer F.Cu) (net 7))
 (segment (start 85.4067 161.2923) (end 85.6545 161.0445) (width 0.25) (layer F.Cu) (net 7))
 (segment (start 85.6545 161.0445) (end 84.139 162.56) (width 0.25) (layer F.Cu) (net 7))
 (segment (start 84.139 166.051) (end 82.55 167.64) (width 0.25) (layer F.Cu) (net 7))
 (segment (start 84.139 162.56) (end 84.139 166.051) (width 0.25) (layer F.Cu) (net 7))
 (segment (start 87.134 183.072) (end 86.134 183.072) (width 0.25) (layer F.Cu) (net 2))
 (segment (start 87.376 182.83) (end 87.134 183.072) (width 0.25) (layer F.Cu) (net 2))
 (segment (start 87.376 179.7535) (end 87.376 182.83) (width 0.25) (layer F.Cu) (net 2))
 (segment (start 113.689 162.6235) (end 113.717 162.5955) (width 0.25) (layer F.Cu) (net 5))
 (segment (start 113.59 164.54) (end 113.59 162.5955) (width 0.25) (layer F.Cu) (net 5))
 (segment (start 81.28 184.15) (end 93.98 184.15) (width 0.25) (layer F.Cu) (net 5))
 (segment (start 67.31 182.88) (end 71.12 179.07) (width 0.25) (layer F.Cu) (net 5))
 (segment (start 76.2 179.07) (end 81.28 184.15) (width 0.25) (layer F.Cu) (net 5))
 (segment (start 71.12 179.07) (end 76.2 179.07) (width 0.25) (layer F.Cu) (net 5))
 (segment (start 93.98 184.15) (end 113.59 164.54) (width 0.25) (layer F.Cu) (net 5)))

